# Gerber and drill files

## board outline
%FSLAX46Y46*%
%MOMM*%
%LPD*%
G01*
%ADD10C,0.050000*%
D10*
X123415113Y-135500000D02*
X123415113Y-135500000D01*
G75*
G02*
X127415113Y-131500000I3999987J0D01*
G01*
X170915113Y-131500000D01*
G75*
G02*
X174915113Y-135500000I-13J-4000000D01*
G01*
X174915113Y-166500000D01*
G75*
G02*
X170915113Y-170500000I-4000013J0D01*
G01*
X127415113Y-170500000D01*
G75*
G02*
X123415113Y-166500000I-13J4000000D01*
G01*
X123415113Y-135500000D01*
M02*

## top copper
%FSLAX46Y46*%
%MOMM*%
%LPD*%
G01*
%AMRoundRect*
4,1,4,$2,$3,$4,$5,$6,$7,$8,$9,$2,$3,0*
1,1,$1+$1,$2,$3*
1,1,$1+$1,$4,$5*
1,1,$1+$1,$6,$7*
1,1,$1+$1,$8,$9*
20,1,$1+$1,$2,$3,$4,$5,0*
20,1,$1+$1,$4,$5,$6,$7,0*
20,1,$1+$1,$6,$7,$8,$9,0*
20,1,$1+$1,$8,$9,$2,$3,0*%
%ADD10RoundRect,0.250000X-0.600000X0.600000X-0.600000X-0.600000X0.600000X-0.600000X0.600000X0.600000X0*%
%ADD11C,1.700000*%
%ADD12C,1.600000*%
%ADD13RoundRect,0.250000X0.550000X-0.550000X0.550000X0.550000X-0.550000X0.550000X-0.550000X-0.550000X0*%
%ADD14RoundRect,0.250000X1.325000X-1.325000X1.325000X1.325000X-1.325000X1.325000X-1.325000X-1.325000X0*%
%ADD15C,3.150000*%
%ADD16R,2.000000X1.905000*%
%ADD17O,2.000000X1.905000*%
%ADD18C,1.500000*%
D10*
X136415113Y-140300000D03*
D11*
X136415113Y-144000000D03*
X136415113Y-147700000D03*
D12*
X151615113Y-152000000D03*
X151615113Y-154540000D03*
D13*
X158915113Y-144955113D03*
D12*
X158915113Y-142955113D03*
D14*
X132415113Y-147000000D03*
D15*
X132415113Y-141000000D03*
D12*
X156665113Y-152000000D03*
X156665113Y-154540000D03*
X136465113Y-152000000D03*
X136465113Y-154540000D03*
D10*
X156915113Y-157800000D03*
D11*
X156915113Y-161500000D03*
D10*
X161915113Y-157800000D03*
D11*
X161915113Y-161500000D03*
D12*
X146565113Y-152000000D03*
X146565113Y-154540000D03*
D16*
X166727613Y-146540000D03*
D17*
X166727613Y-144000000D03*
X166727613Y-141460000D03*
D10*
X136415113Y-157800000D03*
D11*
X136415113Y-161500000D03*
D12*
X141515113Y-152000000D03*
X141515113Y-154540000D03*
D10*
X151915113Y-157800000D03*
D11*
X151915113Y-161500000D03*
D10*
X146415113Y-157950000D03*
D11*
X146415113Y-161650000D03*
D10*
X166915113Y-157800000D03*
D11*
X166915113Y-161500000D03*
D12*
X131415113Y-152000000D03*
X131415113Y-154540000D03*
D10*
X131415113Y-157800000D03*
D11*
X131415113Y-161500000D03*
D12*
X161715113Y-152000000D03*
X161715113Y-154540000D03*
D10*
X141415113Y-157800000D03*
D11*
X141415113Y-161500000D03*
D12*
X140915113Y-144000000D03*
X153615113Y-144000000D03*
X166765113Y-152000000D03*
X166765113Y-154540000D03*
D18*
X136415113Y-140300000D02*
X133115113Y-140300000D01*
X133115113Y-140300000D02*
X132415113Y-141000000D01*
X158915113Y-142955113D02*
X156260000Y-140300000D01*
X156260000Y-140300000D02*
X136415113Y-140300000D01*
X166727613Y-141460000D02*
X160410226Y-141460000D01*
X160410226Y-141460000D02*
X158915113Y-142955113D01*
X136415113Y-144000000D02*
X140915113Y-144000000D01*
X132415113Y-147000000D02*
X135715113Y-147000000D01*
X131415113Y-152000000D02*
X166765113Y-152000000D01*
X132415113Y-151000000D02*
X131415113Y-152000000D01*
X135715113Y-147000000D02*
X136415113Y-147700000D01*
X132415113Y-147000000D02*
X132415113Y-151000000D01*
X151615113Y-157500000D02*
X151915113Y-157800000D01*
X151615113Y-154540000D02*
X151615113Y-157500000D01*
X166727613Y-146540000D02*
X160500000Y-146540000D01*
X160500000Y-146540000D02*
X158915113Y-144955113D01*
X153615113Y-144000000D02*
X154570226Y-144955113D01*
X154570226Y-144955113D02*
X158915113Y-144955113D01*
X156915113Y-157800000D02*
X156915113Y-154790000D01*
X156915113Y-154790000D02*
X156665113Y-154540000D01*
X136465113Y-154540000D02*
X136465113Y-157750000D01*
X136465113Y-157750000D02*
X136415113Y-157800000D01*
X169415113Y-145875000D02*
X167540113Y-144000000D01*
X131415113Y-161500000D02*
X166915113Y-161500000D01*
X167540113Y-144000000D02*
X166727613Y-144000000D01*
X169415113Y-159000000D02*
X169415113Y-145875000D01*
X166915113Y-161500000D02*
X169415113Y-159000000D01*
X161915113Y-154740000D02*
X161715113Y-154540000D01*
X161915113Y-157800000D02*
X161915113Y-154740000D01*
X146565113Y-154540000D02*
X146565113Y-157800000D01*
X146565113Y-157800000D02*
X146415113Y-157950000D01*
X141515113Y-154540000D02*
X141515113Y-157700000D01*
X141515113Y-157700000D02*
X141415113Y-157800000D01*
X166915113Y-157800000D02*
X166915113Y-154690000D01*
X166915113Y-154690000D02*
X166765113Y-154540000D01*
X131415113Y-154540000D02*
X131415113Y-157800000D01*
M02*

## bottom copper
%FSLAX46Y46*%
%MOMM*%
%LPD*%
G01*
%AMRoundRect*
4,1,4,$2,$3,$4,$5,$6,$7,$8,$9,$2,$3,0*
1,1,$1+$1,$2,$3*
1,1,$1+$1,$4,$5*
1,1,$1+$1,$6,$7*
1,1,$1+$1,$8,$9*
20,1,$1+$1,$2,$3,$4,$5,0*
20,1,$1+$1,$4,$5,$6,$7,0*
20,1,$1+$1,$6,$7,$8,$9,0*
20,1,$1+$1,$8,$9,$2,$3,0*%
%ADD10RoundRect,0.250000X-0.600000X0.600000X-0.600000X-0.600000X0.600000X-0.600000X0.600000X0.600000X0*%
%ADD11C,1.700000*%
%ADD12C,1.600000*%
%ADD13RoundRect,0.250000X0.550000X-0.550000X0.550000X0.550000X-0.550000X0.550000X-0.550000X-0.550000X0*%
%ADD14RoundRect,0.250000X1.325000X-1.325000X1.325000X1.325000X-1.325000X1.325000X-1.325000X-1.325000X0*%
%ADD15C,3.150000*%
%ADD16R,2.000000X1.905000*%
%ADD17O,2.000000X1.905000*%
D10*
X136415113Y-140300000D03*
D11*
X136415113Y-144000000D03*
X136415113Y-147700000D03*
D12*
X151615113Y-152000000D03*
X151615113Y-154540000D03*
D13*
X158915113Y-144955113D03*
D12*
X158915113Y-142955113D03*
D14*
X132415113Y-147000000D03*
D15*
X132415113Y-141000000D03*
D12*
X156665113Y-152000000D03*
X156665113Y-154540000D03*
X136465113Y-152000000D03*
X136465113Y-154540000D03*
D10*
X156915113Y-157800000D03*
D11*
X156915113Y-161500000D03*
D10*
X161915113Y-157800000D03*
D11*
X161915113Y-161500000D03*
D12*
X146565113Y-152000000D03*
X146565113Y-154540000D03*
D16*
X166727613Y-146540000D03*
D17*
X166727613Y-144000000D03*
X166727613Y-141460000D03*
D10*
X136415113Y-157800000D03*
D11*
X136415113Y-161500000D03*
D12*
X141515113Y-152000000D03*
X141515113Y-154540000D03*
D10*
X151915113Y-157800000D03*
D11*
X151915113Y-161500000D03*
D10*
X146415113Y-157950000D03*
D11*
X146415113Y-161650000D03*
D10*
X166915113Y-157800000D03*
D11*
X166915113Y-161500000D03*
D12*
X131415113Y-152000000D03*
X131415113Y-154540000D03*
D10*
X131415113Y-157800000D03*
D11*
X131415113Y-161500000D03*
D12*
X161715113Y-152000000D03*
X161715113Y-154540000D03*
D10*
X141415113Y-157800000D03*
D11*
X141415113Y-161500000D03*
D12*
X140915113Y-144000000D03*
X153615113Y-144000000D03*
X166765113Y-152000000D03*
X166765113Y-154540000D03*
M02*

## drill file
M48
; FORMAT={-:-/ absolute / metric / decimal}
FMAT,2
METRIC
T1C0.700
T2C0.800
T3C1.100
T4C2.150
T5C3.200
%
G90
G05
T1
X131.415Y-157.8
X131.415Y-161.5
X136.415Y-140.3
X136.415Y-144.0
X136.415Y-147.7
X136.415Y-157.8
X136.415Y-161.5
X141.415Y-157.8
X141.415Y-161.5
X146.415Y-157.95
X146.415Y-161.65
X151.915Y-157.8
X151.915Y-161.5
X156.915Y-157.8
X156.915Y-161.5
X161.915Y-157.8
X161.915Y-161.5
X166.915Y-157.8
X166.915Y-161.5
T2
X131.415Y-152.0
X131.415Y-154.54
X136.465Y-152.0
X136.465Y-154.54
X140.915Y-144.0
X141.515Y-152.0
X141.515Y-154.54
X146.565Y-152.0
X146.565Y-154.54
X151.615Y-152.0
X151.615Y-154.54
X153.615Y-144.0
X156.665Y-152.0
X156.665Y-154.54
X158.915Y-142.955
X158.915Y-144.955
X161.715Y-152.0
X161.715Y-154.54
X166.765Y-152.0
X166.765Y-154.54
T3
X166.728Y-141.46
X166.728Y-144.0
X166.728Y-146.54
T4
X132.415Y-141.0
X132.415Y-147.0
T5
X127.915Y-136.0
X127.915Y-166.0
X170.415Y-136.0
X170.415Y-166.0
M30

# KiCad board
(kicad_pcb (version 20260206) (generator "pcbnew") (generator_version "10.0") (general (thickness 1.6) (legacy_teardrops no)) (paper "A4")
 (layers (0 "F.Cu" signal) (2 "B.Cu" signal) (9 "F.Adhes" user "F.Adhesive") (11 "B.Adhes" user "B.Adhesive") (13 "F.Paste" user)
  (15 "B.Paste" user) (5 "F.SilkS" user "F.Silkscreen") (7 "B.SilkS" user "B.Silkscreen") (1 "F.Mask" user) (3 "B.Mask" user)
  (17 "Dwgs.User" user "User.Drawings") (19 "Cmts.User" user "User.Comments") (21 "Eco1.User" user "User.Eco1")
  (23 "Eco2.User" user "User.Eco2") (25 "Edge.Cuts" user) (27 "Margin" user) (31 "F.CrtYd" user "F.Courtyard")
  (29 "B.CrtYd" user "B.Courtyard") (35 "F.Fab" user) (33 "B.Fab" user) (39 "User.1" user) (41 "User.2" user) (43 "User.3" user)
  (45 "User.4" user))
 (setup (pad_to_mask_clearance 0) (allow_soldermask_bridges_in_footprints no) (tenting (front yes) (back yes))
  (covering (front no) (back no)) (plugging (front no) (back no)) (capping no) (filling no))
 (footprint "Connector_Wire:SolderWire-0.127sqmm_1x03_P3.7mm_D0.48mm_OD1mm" (layer "F.Cu") (at 136.415113 140.3 -90)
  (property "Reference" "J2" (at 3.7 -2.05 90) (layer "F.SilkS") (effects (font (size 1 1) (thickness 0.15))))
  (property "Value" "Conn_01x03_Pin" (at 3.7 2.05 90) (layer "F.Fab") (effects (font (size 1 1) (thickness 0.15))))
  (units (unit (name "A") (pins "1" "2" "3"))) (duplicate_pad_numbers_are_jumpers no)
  (pad "1" thru_hole roundrect (at 0 0 270) (size 1.7 1.7) (drill 0.7) (layers "*.Cu" "*.Mask") (remove_unused_layers no)
   (roundrect_rratio 0.147059) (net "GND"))
  (pad "2" thru_hole circle (at 3.7 0 270) (size 1.7 1.7) (drill 0.7) (layers "*.Cu" "*.Mask") (remove_unused_layers no)
   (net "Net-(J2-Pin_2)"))
  (pad "3" thru_hole circle (at 7.4 0 270) (size 1.7 1.7) (drill 0.7) (layers "*.Cu" "*.Mask") (remove_unused_layers no) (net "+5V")))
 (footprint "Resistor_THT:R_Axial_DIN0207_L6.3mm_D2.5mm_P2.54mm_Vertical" (layer "F.Cu") (at 151.615113 152 -90)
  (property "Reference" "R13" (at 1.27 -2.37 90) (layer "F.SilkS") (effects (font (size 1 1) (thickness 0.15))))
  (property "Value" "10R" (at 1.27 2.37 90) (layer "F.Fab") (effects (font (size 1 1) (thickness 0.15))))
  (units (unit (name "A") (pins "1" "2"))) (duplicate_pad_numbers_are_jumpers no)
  (pad "1" thru_hole circle (at 0 0 270) (size 1.6 1.6) (drill 0.8) (layers "*.Cu" "*.Mask") (remove_unused_layers no) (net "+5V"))
  (pad "2" thru_hole circle (at 2.54 0 270) (size 1.6 1.6) (drill 0.8) (layers "*.Cu" "*.Mask") (remove_unused_layers no)
   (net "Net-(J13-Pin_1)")))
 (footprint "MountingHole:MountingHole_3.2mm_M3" (layer "F.Cu") (at 170.415113 136)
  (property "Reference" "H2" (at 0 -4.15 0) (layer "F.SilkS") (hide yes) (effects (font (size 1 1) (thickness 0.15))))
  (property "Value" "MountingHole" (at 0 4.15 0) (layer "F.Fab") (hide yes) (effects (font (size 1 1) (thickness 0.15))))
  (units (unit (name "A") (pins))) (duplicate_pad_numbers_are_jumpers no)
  (pad "" np_thru_hole circle (at 0 0) (size 3.2 3.2) (drill 3.2) (layers "*.Cu" "*.Mask")))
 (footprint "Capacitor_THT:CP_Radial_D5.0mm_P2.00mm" (layer "F.Cu") (at 158.915113 144.955113 90)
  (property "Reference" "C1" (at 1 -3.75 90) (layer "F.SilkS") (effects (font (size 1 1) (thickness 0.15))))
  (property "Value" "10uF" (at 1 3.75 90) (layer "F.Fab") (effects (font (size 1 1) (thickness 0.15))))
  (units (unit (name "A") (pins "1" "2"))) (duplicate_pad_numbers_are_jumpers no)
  (pad "1" thru_hole roundrect (at 0 0 90) (size 1.6 1.6) (drill 0.8) (layers "*.Cu" "*.Mask") (remove_unused_layers no)
   (roundrect_rratio 0.15625) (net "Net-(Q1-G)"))
  (pad "2" thru_hole circle (at 2 0 90) (size 1.6 1.6) (drill 0.8) (layers "*.Cu" "*.Mask") (remove_unused_layers no) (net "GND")))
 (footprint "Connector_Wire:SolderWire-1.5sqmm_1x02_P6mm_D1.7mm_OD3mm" (layer "F.Cu") (at 132.415113 147 90)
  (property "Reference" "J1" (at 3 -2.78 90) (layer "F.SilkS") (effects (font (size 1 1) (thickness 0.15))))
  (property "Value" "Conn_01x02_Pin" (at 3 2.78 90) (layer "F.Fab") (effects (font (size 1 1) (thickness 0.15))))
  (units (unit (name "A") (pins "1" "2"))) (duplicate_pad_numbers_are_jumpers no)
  (pad "1" thru_hole roundrect (at 0 0 90) (size 3.15 3.15) (drill 2.15) (layers "*.Cu" "*.Mask") (remove_unused_layers no)
   (roundrect_rratio 0.079365) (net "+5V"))
  (pad "2" thru_hole circle (at 6 0 90) (size 3.15 3.15) (drill 2.15) (layers "*.Cu" "*.Mask") (remove_unused_layers no) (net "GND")))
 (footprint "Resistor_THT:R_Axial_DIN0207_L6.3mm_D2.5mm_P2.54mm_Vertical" (layer "F.Cu") (at 156.665113 152 -90)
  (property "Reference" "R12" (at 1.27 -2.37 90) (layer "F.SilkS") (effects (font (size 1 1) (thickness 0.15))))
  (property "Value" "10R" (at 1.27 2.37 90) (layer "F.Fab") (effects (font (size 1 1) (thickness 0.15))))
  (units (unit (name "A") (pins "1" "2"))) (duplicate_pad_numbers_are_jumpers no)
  (pad "1" thru_hole circle (at 0 0 270) (size 1.6 1.6) (drill 0.8) (layers "*.Cu" "*.Mask") (remove_unused_layers no) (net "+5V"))
  (pad "2" thru_hole circle (at 2.54 0 270) (size 1.6 1.6) (drill 0.8) (layers "*.Cu" "*.Mask") (remove_unused_layers no)
   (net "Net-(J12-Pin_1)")))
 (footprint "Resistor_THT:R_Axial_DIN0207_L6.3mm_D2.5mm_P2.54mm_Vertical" (layer "F.Cu") (at 136.465113 152 -90)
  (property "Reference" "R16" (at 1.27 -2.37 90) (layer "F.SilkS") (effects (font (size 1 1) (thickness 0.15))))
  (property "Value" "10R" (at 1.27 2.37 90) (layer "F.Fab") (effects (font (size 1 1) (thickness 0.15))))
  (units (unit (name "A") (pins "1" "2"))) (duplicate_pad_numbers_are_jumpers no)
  (pad "1" thru_hole circle (at 0 0 270) (size 1.6 1.6) (drill 0.8) (layers "*.Cu" "*.Mask") (remove_unused_layers no) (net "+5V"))
  (pad "2" thru_hole circle (at 2.54 0 270) (size 1.6 1.6) (drill 0.8) (layers "*.Cu" "*.Mask") (remove_unused_layers no)
   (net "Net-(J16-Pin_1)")))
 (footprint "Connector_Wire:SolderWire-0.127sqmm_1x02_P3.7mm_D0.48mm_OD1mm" (layer "F.Cu") (at 156.915113 157.8 -90)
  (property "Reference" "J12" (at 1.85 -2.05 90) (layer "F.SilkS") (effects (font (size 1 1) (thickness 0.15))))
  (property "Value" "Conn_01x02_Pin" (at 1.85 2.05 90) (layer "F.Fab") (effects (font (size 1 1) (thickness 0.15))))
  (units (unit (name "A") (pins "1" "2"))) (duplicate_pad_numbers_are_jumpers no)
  (pad "1" thru_hole roundrect (at 0 0 270) (size 1.7 1.7) (drill 0.7) (layers "*.Cu" "*.Mask") (remove_unused_layers no)
   (roundrect_rratio 0.147059) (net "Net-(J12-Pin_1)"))
  (pad "2" thru_hole circle (at 3.7 0 270) (size 1.7 1.7) (drill 0.7) (layers "*.Cu" "*.Mask") (remove_unused_layers no)
   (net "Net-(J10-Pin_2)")))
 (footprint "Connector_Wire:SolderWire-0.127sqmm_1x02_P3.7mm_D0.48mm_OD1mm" (layer "F.Cu") (at 161.915113 157.8 -90)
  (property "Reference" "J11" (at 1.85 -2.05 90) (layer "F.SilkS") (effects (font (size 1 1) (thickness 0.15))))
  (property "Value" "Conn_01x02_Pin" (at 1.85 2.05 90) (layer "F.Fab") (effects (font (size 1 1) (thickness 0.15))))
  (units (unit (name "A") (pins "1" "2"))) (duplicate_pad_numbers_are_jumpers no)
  (pad "1" thru_hole roundrect (at 0 0 270) (size 1.7 1.7) (drill 0.7) (layers "*.Cu" "*.Mask") (remove_unused_layers no)
   (roundrect_rratio 0.147059) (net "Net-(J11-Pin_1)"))
  (pad "2" thru_hole circle (at 3.7 0 270) (size 1.7 1.7) (drill 0.7) (layers "*.Cu" "*.Mask") (remove_unused_layers no)
   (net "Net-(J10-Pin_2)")))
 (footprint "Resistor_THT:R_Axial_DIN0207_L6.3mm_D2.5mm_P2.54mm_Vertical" (layer "F.Cu") (at 146.565113 152 -90)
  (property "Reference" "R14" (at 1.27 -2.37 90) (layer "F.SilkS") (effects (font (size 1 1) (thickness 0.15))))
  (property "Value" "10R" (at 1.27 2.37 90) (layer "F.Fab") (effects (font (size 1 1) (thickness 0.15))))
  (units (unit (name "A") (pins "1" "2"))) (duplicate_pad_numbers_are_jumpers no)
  (pad "1" thru_hole circle (at 0 0 270) (size 1.6 1.6) (drill 0.8) (layers "*.Cu" "*.Mask") (remove_unused_layers no) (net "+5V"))
  (pad "2" thru_hole circle (at 2.54 0 270) (size 1.6 1.6) (drill 0.8) (layers "*.Cu" "*.Mask") (remove_unused_layers no)
   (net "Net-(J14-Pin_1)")))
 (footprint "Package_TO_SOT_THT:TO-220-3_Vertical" (layer "F.Cu") (at 166.727613 146.54 90)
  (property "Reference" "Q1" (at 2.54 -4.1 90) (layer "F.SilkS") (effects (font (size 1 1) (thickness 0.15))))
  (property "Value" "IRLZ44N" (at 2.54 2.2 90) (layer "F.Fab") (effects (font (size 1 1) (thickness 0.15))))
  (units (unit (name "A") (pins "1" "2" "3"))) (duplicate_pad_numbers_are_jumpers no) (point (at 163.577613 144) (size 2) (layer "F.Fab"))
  (pad "1" thru_hole rect (at 0 0 90) (size 1.905 2) (drill 1.1) (layers "*.Cu" "*.Mask") (remove_unused_layers no) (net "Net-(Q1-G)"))
  (pad "2" thru_hole oval (at 2.54 0 90) (size 1.905 2) (drill 1.1) (layers "*.Cu" "*.Mask") (remove_unused_layers no)
   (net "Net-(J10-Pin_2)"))
  (pad "3" thru_hole oval (at 5.08 0 90) (size 1.905 2) (drill 1.1) (layers "*.Cu" "*.Mask") (remove_unused_layers no) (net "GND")))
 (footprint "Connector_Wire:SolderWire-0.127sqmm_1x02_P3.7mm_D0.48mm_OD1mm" (layer "F.Cu") (at 136.415113 157.8 -90)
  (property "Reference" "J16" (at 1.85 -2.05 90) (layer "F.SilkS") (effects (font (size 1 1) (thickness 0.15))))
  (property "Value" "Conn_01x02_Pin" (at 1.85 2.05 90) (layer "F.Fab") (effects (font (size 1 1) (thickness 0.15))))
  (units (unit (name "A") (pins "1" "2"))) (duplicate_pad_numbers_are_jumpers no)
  (pad "1" thru_hole roundrect (at 0 0 270) (size 1.7 1.7) (drill 0.7) (layers "*.Cu" "*.Mask") (remove_unused_layers no)
   (roundrect_rratio 0.147059) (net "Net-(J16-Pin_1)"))
  (pad "2" thru_hole circle (at 3.7 0 270) (size 1.7 1.7) (drill 0.7) (layers "*.Cu" "*.Mask") (remove_unused_layers no)
   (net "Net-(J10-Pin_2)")))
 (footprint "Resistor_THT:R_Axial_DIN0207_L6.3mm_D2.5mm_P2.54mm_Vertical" (layer "F.Cu") (at 141.515113 152 -90)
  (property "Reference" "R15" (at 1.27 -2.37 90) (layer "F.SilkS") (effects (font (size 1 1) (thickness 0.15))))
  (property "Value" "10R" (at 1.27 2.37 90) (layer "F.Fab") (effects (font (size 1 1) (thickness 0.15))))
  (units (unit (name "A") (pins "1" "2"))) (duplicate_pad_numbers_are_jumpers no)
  (pad "1" thru_hole circle (at 0 0 270) (size 1.6 1.6) (drill 0.8) (layers "*.Cu" "*.Mask") (remove_unused_layers no) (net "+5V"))
  (pad "2" thru_hole circle (at 2.54 0 270) (size 1.6 1.6) (drill 0.8) (layers "*.Cu" "*.Mask") (remove_unused_layers no)
   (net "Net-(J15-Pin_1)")))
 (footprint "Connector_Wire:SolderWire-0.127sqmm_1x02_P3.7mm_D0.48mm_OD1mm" (layer "F.Cu") (at 151.915113 157.8 -90)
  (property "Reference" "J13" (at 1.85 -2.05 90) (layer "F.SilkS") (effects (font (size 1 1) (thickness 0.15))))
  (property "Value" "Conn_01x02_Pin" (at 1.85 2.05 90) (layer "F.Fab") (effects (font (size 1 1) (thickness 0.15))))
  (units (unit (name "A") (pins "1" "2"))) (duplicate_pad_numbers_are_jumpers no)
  (pad "1" thru_hole roundrect (at 0 0 270) (size 1.7 1.7) (drill 0.7) (layers "*.Cu" "*.Mask") (remove_unused_layers no)
   (roundrect_rratio 0.147059) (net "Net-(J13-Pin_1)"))
  (pad "2" thru_hole circle (at 3.7 0 270) (size 1.7 1.7) (drill 0.7) (layers "*.Cu" "*.Mask") (remove_unused_layers no)
   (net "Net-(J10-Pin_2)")))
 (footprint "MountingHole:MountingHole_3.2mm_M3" (layer "F.Cu") (at 127.915113 136)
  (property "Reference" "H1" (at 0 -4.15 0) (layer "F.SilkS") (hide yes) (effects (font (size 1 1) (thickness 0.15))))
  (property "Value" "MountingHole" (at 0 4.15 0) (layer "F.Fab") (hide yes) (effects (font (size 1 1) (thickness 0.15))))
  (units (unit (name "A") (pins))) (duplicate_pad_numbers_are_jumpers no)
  (pad "" np_thru_hole circle (at 0 0) (size 3.2 3.2) (drill 3.2) (layers "*.Cu" "*.Mask")))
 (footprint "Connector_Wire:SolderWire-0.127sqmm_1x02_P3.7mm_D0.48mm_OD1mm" (layer "F.Cu") (at 146.415113 157.95 -90)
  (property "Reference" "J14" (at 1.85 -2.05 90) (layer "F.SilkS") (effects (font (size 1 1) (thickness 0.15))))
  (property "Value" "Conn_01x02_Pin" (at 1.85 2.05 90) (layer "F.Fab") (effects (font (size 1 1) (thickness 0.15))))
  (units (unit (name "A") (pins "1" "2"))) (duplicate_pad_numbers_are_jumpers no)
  (pad "1" thru_hole roundrect (at 0 0 270) (size 1.7 1.7) (drill 0.7) (layers "*.Cu" "*.Mask") (remove_unused_layers no)
   (roundrect_rratio 0.147059) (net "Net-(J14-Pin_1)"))
  (pad "2" thru_hole circle (at 3.7 0 270) (size 1.7 1.7) (drill 0.7) (layers "*.Cu" "*.Mask") (remove_unused_layers no)
   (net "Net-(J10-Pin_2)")))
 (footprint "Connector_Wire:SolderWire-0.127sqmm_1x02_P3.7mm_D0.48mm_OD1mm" (layer "F.Cu") (at 166.915113 157.8 -90)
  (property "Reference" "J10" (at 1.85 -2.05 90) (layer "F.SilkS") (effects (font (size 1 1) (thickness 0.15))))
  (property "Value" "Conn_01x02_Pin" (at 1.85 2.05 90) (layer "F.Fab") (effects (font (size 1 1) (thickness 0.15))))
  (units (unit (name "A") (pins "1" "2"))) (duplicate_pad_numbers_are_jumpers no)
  (pad "1" thru_hole roundrect (at 0 0 270) (size 1.7 1.7) (drill 0.7) (layers "*.Cu" "*.Mask") (remove_unused_layers no)
   (roundrect_rratio 0.147059) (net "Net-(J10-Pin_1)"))
  (pad "2" thru_hole circle (at 3.7 0 270) (size 1.7 1.7) (drill 0.7) (layers "*.Cu" "*.Mask") (remove_unused_layers no)
   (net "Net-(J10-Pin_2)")))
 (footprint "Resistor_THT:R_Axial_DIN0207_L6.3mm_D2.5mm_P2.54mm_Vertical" (layer "F.Cu") (at 131.415113 152 -90)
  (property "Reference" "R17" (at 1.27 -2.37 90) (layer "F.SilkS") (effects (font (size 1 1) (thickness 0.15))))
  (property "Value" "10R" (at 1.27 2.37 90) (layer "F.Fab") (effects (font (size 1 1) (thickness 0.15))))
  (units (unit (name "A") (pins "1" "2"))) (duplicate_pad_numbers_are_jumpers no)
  (pad "1" thru_hole circle (at 0 0 270) (size 1.6 1.6) (drill 0.8) (layers "*.Cu" "*.Mask") (remove_unused_layers no) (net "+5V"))
  (pad "2" thru_hole circle (at 2.54 0 270) (size 1.6 1.6) (drill 0.8) (layers "*.Cu" "*.Mask") (remove_unused_layers no)
   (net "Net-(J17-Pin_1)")))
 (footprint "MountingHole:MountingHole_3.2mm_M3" (layer "F.Cu") (at 127.915113 166)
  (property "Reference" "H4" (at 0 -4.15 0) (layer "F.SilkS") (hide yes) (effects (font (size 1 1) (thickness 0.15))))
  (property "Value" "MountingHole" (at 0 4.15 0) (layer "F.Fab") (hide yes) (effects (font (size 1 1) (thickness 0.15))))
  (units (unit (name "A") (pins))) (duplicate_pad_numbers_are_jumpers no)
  (pad "" np_thru_hole circle (at 0 0) (size 3.2 3.2) (drill 3.2) (layers "*.Cu" "*.Mask")))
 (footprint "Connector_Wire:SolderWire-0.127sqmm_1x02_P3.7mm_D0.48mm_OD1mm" (layer "F.Cu") (at 131.415113 157.8 -90)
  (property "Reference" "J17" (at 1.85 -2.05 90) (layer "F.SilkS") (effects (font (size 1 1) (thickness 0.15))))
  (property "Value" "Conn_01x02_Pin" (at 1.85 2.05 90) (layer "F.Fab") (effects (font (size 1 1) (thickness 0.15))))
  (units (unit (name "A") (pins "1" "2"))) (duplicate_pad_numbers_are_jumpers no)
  (pad "1" thru_hole roundrect (at 0 0 270) (size 1.7 1.7) (drill 0.7) (layers "*.Cu" "*.Mask") (remove_unused_layers no)
   (roundrect_rratio 0.147059) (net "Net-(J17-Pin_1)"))
  (pad "2" thru_hole circle (at 3.7 0 270) (size 1.7 1.7) (drill 0.7) (layers "*.Cu" "*.Mask") (remove_unused_layers no)
   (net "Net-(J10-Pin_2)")))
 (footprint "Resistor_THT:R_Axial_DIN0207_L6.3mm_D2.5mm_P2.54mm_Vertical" (layer "F.Cu") (at 161.715113 152 -90)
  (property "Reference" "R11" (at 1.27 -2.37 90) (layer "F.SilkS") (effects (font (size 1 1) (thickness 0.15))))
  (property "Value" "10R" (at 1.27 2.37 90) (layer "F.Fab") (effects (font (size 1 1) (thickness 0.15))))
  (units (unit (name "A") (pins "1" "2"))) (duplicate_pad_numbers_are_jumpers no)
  (pad "1" thru_hole circle (at 0 0 270) (size 1.6 1.6) (drill 0.8) (layers "*.Cu" "*.Mask") (remove_unused_layers no) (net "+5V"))
  (pad "2" thru_hole circle (at 2.54 0 270) (size 1.6 1.6) (drill 0.8) (layers "*.Cu" "*.Mask") (remove_unused_layers no)
   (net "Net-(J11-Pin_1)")))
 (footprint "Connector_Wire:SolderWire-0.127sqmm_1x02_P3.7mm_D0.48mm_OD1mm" (layer "F.Cu") (at 141.415113 157.8 -90)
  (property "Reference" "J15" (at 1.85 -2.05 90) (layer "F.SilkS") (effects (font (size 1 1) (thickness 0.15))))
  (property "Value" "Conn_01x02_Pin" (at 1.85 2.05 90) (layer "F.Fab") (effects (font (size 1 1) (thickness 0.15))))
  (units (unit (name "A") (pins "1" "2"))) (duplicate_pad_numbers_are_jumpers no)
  (pad "1" thru_hole roundrect (at 0 0 270) (size 1.7 1.7) (drill 0.7) (layers "*.Cu" "*.Mask") (remove_unused_layers no)
   (roundrect_rratio 0.147059) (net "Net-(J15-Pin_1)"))
  (pad "2" thru_hole circle (at 3.7 0 270) (size 1.7 1.7) (drill 0.7) (layers "*.Cu" "*.Mask") (remove_unused_layers no)
   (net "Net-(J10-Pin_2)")))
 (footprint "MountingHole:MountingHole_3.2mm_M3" (layer "F.Cu") (at 170.415113 166)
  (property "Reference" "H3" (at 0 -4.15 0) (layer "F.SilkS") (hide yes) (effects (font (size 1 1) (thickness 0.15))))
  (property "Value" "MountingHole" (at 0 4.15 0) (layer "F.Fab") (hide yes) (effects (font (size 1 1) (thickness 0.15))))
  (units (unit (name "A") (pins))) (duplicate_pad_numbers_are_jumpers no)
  (pad "" np_thru_hole circle (at 0 0) (size 3.2 3.2) (drill 3.2) (layers "*.Cu" "*.Mask")))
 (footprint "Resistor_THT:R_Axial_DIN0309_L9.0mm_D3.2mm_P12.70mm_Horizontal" (layer "F.Cu") (at 140.915113 144)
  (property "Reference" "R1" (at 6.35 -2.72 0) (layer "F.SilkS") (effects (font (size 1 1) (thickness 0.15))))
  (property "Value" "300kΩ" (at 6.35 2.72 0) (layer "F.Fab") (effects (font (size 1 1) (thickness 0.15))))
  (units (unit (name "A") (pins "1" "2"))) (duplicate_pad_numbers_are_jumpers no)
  (pad "1" thru_hole circle (at 0 0) (size 1.6 1.6) (drill 0.8) (layers "*.Cu" "*.Mask") (remove_unused_layers no) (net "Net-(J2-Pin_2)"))
  (pad "2" thru_hole circle (at 12.7 0) (size 1.6 1.6) (drill 0.8) (layers "*.Cu" "*.Mask") (remove_unused_layers no) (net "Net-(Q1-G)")))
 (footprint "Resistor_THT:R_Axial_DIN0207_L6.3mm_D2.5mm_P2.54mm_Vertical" (layer "F.Cu") (at 166.765113 152 -90)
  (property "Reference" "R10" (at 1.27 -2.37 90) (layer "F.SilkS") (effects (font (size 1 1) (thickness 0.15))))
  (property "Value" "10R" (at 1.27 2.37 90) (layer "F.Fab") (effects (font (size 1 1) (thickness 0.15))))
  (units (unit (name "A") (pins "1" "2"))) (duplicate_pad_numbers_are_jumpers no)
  (pad "1" thru_hole circle (at 0 0 270) (size 1.6 1.6) (drill 0.8) (layers "*.Cu" "*.Mask") (remove_unused_layers no) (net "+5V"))
  (pad "2" thru_hole circle (at 2.54 0 270) (size 1.6 1.6) (drill 0.8) (layers "*.Cu" "*.Mask") (remove_unused_layers no)
   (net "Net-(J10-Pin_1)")))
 (gr_rect (start 123.415113 131.5) (end 174.915113 170.5) (radius 4) (stroke (width 0.05) (type solid)) (fill no) (layer "Edge.Cuts"))
 (segment (start 136.415113 140.3) (end 133.115113 140.3) (width 1.5) (layer "F.Cu") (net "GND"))
 (segment (start 133.115113 140.3) (end 132.415113 141) (width 1.5) (layer "F.Cu") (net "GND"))
 (segment (start 158.915113 142.955113) (end 156.26 140.3) (width 1.5) (layer "F.Cu") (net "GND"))
 (segment (start 156.26 140.3) (end 136.415113 140.3) (width 1.5) (layer "F.Cu") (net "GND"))
 (segment (start 166.727613 141.46) (end 160.410226 141.46) (width 1.5) (layer "F.Cu") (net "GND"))
 (segment (start 160.410226 141.46) (end 158.915113 142.955113) (width 1.5) (layer "F.Cu") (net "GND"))
 (segment (start 136.415113 144) (end 140.915113 144) (width 1.5) (layer "F.Cu") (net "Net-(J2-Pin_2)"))
 (segment (start 132.415113 147) (end 135.715113 147) (width 1.5) (layer "F.Cu") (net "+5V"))
 (segment (start 131.415113 152) (end 166.765113 152) (width 1.5) (layer "F.Cu") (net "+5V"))
 (segment (start 132.415113 151) (end 131.415113 152) (width 1.5) (layer "F.Cu") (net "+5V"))
 (segment (start 135.715113 147) (end 136.415113 147.7) (width 1.5) (layer "F.Cu") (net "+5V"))
 (segment (start 132.415113 147) (end 132.415113 151) (width 1.5) (layer "F.Cu") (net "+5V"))
 (segment (start 151.615113 157.5) (end 151.915113 157.8) (width 1.5) (layer "F.Cu") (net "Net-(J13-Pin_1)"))
 (segment (start 151.615113 154.54) (end 151.615113 157.5) (width 1.5) (layer "F.Cu") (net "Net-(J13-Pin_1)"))
 (segment (start 166.727613 146.54) (end 160.5 146.54) (width 1.5) (layer "F.Cu") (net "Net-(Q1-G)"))
 (segment (start 160.5 146.54) (end 158.915113 144.955113) (width 1.5) (layer "F.Cu") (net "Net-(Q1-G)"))
 (segment (start 153.615113 144) (end 154.570226 144.955113) (width 1.5) (layer "F.Cu") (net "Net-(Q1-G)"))
 (segment (start 154.570226 144.955113) (end 158.915113 144.955113) (width 1.5) (layer "F.Cu") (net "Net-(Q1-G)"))
 (segment (start 156.915113 157.8) (end 156.915113 154.79) (width 1.5) (layer "F.Cu") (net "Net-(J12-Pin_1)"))
 (segment (start 156.915113 154.79) (end 156.665113 154.54) (width 1.5) (layer "F.Cu") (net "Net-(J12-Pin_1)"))
 (segment (start 136.465113 154.54) (end 136.465113 157.75) (width 1.5) (layer "F.Cu") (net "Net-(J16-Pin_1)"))
 (segment (start 136.465113 157.75) (end 136.415113 157.8) (width 1.5) (layer "F.Cu") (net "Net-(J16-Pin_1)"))
 (segment (start 169.415113 145.875) (end 167.540113 144) (width 1.5) (layer "F.Cu") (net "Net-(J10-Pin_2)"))
 (segment (start 131.415113 161.5) (end 166.915113 161.5) (width 1.5) (layer "F.Cu") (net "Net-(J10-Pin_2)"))
 (segment (start 167.540113 144) (end 166.727613 144) (width 1.5) (layer "F.Cu") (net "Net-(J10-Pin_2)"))
 (segment (start 169.415113 159) (end 169.415113 145.875) (width 1.5) (layer "F.Cu") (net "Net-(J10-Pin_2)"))
 (segment (start 166.915113 161.5) (end 169.415113 159) (width 1.5) (layer "F.Cu") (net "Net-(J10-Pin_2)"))
 (segment (start 161.915113 154.74) (end 161.715113 154.54) (width 1.5) (layer "F.Cu") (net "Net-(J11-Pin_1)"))
 (segment (start 161.915113 157.8) (end 161.915113 154.74) (width 1.5) (layer "F.Cu") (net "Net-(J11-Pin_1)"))
 (segment (start 146.565113 154.54) (end 146.565113 157.8) (width 1.5) (layer "F.Cu") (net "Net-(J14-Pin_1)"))
 (segment (start 146.565113 157.8) (end 146.415113 157.95) (width 1.5) (layer "F.Cu") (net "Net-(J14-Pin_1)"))
 (segment (start 141.515113 154.54) (end 141.515113 157.7) (width 1.5) (layer "F.Cu") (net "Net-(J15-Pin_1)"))
 (segment (start 141.515113 157.7) (end 141.415113 157.8) (width 1.5) (layer "F.Cu") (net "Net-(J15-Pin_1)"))
 (segment (start 166.915113 157.8) (end 166.915113 154.69) (width 1.5) (layer "F.Cu") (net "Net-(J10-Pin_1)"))
 (segment (start 166.915113 154.69) (end 166.765113 154.54) (width 1.5) (layer "F.Cu") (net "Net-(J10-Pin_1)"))
 (segment (start 131.415113 154.54) (end 131.415113 157.8) (width 1.5) (layer "F.Cu") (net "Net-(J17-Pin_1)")))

